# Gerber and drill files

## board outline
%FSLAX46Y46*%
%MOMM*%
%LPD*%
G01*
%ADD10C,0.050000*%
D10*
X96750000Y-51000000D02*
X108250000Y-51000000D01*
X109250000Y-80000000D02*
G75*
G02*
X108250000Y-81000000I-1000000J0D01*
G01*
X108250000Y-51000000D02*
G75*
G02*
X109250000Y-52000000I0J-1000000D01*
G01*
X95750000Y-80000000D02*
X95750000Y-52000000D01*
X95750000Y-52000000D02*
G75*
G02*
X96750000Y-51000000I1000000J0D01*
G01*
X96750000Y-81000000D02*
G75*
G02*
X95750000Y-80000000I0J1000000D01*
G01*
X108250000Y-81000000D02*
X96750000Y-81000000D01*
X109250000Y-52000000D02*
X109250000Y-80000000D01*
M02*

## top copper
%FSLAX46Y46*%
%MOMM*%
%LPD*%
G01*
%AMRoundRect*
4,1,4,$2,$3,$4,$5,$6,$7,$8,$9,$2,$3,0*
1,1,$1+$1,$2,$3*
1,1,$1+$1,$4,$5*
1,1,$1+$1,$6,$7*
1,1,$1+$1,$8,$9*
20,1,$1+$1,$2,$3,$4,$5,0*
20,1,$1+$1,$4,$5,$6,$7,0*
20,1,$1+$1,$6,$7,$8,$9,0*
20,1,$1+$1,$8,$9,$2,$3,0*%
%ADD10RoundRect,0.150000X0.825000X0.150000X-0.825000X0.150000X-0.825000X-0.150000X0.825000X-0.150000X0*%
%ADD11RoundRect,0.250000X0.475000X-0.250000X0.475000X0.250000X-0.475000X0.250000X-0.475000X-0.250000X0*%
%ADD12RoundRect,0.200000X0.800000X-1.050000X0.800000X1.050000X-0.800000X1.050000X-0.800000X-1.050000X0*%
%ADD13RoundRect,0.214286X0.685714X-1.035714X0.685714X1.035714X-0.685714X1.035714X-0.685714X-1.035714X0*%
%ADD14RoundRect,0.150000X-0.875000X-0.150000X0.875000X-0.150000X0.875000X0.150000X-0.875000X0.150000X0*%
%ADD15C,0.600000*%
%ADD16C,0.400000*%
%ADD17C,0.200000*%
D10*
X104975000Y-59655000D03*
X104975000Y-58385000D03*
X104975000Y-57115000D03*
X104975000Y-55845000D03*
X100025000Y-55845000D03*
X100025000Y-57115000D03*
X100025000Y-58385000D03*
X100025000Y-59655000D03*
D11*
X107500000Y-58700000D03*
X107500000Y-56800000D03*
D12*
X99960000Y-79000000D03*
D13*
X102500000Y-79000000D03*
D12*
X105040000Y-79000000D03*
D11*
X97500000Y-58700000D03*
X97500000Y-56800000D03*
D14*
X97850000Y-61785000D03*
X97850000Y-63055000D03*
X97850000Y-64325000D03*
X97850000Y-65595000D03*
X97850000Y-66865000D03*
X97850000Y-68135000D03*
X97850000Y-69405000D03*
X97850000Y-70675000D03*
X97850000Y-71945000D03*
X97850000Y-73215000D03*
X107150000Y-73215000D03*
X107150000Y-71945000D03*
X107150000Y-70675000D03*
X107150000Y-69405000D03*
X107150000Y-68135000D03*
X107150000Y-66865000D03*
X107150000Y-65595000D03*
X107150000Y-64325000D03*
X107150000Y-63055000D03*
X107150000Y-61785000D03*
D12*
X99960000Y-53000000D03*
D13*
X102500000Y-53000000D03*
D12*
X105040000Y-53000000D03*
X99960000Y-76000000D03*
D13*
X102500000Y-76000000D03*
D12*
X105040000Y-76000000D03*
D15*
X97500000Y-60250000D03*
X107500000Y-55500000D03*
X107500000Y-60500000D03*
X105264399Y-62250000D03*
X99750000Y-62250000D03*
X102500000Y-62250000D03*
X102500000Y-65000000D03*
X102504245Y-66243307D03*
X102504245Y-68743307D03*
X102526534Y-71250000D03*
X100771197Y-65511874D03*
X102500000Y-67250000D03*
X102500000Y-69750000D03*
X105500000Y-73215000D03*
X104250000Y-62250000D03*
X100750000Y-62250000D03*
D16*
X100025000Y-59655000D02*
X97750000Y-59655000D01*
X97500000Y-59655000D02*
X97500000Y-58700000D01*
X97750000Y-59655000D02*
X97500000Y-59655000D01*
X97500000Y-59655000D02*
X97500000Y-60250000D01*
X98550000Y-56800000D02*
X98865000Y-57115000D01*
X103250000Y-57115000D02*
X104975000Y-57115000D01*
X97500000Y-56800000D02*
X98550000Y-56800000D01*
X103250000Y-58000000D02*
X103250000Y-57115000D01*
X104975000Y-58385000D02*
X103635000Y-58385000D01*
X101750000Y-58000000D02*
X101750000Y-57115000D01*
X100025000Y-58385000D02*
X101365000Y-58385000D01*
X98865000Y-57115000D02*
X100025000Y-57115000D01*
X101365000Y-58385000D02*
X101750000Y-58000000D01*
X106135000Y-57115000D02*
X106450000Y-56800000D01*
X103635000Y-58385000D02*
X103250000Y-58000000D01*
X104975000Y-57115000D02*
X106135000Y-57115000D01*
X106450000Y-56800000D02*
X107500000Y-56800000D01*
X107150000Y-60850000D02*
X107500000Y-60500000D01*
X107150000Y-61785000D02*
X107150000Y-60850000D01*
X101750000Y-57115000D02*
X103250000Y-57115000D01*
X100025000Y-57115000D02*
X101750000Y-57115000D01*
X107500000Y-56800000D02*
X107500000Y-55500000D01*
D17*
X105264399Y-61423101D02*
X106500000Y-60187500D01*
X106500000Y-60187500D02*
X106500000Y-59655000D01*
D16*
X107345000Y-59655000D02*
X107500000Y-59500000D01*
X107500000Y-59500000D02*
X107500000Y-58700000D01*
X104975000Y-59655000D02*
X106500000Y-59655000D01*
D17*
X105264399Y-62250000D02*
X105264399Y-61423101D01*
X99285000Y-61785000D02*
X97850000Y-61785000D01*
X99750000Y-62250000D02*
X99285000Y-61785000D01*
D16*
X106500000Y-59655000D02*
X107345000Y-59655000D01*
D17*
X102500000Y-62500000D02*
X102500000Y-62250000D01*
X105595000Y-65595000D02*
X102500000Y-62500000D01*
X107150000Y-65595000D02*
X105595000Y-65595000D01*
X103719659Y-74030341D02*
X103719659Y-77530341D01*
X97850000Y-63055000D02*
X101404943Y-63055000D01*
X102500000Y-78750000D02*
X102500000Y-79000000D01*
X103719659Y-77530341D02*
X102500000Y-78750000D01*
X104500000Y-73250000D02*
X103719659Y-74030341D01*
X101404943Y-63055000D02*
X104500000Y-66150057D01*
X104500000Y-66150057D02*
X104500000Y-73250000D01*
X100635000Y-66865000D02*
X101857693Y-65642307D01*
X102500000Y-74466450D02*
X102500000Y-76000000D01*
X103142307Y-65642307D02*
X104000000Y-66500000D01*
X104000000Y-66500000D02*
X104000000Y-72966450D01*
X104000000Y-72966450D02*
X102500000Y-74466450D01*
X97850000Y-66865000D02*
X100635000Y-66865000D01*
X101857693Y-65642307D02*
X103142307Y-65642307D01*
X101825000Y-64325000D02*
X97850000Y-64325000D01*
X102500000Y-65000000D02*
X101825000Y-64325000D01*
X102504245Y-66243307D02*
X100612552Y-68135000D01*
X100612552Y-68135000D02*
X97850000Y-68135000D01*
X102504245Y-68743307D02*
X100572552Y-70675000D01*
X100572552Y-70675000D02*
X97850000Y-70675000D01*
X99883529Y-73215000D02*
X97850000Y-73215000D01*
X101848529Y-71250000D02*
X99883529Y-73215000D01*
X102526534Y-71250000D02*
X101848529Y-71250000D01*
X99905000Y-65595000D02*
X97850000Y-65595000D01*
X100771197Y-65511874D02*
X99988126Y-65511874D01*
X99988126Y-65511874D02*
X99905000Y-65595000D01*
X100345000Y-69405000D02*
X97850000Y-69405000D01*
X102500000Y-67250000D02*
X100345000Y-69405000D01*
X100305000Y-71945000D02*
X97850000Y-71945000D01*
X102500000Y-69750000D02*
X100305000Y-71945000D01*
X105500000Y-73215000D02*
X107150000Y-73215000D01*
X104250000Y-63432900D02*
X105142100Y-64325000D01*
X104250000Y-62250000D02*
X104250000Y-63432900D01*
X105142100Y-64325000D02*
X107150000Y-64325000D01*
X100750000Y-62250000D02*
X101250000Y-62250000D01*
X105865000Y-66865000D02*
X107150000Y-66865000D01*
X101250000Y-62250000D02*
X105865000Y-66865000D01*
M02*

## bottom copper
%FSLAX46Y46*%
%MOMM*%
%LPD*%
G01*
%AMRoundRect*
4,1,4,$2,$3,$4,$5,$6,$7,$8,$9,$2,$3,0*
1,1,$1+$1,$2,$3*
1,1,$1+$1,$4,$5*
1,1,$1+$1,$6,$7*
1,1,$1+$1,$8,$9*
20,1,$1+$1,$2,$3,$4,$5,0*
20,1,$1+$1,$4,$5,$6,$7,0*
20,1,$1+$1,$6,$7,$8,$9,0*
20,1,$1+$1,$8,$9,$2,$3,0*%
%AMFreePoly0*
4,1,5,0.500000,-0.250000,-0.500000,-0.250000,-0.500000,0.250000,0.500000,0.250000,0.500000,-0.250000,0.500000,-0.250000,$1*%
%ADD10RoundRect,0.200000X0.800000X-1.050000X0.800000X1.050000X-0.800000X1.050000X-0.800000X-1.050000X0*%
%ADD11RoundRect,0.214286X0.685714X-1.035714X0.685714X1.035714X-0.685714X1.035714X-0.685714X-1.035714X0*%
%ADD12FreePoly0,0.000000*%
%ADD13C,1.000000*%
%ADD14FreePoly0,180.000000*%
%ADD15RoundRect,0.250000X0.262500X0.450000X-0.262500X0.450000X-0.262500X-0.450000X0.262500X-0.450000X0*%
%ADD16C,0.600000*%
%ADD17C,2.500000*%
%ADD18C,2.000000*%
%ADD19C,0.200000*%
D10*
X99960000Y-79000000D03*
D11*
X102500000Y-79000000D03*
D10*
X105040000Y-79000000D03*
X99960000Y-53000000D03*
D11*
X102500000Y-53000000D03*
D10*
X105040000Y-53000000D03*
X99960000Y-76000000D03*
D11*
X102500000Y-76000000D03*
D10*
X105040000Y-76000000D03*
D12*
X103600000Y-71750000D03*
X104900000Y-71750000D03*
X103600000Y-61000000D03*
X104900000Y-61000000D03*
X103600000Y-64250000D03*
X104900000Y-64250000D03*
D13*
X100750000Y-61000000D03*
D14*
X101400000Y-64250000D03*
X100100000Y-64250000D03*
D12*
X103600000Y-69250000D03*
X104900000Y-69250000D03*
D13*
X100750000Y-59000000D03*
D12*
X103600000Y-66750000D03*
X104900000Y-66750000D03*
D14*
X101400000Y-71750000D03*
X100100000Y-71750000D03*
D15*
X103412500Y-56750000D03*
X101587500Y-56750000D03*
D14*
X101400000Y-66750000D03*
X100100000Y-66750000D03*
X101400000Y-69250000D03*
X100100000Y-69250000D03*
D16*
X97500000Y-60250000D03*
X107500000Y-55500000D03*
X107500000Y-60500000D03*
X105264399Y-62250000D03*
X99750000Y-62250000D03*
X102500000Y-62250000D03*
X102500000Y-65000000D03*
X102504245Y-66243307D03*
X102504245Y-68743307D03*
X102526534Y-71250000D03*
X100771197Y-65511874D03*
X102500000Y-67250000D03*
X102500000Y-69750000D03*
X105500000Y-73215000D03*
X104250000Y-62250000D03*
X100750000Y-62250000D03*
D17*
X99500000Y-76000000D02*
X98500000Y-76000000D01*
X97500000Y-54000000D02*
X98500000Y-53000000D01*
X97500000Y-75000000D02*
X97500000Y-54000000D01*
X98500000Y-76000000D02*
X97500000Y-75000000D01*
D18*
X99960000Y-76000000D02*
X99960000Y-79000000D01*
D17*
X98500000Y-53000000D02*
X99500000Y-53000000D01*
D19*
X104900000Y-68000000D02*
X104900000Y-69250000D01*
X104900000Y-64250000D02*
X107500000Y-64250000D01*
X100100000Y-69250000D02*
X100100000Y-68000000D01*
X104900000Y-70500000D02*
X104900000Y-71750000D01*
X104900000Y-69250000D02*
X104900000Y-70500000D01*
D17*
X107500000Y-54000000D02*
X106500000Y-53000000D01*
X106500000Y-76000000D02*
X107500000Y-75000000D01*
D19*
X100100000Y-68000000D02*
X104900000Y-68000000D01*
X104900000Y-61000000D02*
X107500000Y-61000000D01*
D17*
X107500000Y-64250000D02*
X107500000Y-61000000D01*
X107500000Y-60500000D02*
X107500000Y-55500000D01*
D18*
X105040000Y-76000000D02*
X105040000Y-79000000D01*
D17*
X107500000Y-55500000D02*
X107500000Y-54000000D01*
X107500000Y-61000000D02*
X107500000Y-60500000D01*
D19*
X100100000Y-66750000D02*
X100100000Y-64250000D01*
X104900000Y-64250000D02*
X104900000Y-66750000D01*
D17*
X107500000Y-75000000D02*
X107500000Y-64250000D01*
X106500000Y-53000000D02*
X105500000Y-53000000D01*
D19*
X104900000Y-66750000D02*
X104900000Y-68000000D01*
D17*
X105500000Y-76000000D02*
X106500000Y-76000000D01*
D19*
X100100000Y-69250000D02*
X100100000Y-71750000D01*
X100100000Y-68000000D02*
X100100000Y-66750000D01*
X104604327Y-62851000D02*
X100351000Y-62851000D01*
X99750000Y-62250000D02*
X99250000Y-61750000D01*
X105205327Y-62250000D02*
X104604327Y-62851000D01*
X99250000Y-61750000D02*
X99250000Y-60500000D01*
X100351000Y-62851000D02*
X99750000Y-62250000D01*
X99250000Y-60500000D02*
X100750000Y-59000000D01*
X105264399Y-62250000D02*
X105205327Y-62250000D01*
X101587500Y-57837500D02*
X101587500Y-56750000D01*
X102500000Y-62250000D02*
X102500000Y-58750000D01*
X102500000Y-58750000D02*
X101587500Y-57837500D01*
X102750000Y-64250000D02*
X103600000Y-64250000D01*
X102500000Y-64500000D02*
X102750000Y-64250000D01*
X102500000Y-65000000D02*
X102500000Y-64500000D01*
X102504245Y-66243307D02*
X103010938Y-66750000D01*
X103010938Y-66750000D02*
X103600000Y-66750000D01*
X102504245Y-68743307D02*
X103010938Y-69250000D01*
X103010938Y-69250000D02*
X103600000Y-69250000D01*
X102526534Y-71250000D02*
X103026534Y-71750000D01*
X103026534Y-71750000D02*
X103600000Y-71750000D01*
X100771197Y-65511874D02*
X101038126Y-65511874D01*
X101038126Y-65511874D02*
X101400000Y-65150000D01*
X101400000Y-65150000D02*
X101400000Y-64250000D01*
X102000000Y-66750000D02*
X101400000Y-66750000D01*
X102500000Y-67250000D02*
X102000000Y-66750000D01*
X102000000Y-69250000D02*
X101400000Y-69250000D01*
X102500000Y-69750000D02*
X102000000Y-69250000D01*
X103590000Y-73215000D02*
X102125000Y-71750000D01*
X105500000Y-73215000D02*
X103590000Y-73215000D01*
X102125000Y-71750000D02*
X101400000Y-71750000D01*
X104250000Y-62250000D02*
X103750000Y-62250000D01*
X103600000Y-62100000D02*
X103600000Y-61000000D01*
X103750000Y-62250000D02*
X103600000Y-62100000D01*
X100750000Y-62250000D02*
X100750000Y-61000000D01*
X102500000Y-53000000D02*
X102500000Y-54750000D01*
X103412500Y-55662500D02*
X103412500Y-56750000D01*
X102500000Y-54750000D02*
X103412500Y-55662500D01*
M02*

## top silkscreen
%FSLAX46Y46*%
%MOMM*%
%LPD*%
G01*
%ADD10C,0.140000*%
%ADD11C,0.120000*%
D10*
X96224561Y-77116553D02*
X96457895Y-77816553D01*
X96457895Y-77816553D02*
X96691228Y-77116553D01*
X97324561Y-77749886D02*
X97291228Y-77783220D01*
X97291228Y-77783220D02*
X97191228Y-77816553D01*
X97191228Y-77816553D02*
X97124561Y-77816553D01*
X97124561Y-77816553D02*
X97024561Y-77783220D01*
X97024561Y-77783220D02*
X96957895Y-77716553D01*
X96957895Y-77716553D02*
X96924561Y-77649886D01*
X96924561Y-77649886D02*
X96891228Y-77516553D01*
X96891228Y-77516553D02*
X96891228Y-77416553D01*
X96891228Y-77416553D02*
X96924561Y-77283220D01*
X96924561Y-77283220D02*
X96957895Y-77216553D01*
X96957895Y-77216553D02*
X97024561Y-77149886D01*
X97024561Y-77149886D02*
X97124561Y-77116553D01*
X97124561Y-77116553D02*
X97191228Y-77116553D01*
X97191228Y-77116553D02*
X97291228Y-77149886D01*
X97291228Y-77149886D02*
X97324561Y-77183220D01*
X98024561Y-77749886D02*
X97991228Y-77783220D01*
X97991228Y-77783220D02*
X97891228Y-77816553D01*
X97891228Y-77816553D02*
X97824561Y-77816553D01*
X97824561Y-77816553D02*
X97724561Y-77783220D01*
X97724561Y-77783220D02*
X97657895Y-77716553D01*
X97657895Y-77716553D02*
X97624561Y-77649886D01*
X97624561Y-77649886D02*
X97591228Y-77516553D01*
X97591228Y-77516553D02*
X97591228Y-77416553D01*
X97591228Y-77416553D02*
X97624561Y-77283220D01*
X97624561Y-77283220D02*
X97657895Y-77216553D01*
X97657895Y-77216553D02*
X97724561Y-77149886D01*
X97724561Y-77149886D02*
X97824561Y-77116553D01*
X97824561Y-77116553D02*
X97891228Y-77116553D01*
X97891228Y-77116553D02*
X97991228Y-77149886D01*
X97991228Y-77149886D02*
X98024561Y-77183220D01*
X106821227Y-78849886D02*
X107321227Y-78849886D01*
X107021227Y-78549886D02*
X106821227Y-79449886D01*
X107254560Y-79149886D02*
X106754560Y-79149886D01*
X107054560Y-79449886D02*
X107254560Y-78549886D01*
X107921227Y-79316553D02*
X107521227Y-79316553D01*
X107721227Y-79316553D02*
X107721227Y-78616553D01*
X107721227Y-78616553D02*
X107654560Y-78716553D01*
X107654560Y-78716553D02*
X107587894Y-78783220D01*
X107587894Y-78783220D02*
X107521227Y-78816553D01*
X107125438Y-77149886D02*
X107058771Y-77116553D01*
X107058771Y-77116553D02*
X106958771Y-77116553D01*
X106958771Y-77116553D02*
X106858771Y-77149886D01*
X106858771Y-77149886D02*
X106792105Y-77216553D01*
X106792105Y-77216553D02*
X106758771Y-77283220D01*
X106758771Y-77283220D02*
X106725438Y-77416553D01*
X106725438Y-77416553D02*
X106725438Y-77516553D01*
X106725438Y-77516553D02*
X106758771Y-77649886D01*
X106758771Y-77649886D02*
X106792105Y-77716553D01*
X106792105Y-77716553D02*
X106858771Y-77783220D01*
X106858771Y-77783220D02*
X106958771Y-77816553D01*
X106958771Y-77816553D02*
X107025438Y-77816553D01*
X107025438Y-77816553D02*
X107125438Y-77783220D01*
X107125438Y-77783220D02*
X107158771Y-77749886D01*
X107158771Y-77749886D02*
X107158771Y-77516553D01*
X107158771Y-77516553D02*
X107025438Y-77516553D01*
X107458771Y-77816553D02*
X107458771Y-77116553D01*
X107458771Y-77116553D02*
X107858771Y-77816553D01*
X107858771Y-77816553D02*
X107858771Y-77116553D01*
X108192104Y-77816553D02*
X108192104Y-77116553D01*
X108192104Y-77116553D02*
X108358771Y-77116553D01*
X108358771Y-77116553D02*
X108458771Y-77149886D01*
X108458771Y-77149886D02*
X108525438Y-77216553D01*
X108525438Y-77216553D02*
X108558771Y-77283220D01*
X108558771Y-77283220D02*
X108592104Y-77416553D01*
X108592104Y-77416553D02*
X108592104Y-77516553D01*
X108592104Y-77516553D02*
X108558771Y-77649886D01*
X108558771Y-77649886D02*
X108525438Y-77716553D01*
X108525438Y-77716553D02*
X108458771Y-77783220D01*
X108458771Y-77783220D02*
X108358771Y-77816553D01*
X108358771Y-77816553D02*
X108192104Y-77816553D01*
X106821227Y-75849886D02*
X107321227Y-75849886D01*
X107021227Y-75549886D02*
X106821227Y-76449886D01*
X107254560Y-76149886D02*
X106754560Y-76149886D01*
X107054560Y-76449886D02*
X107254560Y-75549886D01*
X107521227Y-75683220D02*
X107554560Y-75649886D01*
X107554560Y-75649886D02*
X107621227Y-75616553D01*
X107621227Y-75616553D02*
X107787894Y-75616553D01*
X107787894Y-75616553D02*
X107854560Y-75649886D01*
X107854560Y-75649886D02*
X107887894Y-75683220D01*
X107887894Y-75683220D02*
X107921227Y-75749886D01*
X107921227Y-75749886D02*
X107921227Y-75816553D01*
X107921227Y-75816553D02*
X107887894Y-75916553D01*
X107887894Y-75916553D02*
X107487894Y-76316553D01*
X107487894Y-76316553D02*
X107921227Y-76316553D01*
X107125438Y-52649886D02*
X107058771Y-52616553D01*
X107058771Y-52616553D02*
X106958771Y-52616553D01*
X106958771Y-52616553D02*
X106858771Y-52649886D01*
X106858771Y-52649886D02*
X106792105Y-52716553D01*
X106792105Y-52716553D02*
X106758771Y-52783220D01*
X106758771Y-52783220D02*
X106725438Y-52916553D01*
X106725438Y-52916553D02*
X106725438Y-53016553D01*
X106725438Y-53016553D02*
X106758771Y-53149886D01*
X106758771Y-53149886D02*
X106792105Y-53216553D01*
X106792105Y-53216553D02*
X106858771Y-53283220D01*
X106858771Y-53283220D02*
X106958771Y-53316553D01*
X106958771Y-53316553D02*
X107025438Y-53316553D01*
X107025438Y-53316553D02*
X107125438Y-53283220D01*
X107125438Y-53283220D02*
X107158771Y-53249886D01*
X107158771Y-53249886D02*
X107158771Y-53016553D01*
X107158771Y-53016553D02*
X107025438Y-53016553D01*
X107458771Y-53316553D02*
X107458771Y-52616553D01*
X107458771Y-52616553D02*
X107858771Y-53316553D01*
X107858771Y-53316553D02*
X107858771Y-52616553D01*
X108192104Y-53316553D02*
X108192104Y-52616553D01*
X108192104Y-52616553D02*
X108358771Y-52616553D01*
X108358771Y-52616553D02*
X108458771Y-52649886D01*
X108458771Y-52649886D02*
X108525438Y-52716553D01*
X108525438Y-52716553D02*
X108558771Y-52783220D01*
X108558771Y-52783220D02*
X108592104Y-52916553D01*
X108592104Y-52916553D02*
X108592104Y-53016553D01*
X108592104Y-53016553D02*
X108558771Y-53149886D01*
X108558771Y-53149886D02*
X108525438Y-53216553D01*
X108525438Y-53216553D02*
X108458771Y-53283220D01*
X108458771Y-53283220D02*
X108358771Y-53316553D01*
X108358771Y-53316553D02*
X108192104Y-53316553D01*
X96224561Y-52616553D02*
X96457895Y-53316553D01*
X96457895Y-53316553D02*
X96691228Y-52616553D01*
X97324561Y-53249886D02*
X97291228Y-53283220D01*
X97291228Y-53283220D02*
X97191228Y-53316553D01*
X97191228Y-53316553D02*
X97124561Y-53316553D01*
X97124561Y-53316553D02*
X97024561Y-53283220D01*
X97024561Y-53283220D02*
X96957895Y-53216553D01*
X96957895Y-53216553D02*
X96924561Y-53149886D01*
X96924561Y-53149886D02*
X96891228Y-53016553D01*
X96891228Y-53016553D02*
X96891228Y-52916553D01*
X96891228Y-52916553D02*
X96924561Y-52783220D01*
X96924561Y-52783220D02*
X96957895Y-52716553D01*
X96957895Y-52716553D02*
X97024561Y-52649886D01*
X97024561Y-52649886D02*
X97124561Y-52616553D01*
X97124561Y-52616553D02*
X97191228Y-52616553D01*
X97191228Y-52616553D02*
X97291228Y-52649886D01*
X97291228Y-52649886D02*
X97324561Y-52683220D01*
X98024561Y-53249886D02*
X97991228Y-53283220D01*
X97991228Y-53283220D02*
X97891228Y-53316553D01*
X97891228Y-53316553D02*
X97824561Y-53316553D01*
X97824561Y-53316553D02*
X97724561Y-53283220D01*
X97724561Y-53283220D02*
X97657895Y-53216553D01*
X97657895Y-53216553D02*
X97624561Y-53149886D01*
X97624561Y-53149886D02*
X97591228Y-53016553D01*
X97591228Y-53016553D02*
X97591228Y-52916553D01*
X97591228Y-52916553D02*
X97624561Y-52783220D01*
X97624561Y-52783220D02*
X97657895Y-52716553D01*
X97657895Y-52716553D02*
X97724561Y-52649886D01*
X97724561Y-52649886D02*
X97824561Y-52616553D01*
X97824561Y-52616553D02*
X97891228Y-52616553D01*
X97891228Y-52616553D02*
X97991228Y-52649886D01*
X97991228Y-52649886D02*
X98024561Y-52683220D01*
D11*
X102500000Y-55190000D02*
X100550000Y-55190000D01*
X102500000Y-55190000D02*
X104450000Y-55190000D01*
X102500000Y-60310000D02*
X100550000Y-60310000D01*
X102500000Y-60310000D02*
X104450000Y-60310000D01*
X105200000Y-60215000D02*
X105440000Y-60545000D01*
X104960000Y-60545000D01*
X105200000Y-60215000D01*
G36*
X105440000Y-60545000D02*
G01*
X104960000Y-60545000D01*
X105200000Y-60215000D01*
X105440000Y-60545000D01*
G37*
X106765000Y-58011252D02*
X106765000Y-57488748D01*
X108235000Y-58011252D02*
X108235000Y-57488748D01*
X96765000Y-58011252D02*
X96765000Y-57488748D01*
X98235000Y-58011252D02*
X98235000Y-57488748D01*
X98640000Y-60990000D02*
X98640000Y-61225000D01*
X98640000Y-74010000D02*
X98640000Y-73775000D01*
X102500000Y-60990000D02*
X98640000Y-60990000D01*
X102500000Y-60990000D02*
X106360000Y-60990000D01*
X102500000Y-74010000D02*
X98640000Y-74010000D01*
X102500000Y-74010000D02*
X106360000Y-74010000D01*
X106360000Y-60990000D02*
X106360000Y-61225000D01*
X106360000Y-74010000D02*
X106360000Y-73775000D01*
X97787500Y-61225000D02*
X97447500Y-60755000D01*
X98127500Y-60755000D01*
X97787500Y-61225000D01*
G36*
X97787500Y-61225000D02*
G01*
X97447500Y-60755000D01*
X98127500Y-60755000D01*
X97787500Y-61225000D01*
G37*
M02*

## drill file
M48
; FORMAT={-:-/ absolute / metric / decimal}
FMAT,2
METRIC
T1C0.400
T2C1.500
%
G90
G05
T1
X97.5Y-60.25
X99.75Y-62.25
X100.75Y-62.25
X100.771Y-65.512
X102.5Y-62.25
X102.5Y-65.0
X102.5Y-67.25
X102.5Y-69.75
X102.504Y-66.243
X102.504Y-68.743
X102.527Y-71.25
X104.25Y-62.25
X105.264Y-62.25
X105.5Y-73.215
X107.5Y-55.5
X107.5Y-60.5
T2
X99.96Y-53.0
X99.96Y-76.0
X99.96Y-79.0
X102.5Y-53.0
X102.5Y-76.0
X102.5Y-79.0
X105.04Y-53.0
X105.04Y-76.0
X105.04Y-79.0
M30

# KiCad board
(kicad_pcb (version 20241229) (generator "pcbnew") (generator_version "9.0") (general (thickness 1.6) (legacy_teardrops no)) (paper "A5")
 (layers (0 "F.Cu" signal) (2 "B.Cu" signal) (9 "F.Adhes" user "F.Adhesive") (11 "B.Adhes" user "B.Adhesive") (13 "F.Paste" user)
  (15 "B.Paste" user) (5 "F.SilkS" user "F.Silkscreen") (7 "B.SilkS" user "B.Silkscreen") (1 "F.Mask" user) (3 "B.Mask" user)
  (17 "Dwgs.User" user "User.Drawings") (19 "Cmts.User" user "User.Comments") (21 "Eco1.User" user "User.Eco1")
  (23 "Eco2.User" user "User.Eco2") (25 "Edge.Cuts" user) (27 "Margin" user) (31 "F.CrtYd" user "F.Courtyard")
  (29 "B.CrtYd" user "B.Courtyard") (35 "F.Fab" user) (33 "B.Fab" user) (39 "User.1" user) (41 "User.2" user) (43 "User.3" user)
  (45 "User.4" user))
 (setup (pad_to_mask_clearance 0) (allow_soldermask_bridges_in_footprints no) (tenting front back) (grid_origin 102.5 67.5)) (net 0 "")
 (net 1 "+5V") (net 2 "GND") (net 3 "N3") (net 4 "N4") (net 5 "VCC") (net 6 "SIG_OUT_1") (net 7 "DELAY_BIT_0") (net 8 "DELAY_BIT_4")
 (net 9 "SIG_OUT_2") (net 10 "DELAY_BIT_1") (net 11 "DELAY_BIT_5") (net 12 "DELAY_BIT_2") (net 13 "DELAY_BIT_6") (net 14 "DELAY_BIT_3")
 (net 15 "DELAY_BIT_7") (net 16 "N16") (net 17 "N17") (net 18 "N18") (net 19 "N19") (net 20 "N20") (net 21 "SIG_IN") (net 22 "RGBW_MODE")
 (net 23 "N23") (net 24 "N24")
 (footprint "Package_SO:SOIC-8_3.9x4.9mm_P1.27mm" (layer "F.Cu") (at 102.5 57.75 180)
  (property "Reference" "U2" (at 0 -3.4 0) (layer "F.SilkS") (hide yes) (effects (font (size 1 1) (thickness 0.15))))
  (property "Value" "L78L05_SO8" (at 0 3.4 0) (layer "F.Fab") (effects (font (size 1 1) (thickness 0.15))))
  (fp_line (start 0 2.56) (end 1.95 2.56) (stroke (width 0.12) (type solid)) (layer "F.SilkS"))
  (fp_line (start 0 2.56) (end -1.95 2.56) (stroke (width 0.12) (type solid)) (layer "F.SilkS"))
  (fp_line (start 0 -2.56) (end 1.95 -2.56) (stroke (width 0.12) (type solid)) (layer "F.SilkS"))
  (fp_line (start 0 -2.56) (end -1.95 -2.56) (stroke (width 0.12) (type solid)) (layer "F.SilkS"))
  (fp_poly (pts (xy -2.7 -2.465) (xy -2.94 -2.795) (xy -2.46 -2.795)) (stroke (width 0.12) (type solid)) (fill yes) (layer "F.SilkS"))
  (pad "1" smd roundrect (at -2.475 -1.905 180) (size 1.95 0.6) (layers "F.Cu" "F.Mask" "F.Paste") (roundrect_rratio 0.25) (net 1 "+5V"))
  (pad "2" smd roundrect (at -2.475 -0.635 180) (size 1.95 0.6) (layers "F.Cu" "F.Mask" "F.Paste") (roundrect_rratio 0.25) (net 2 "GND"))
  (pad "3" smd roundrect (at -2.475 0.635 180) (size 1.95 0.6) (layers "F.Cu" "F.Mask" "F.Paste") (roundrect_rratio 0.25) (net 2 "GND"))
  (pad "4" smd roundrect (at -2.475 1.905 180) (size 1.95 0.6) (layers "F.Cu" "F.Mask" "F.Paste") (roundrect_rratio 0.25) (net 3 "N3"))
  (pad "5" smd roundrect (at 2.475 1.905 180) (size 1.95 0.6) (layers "F.Cu" "F.Mask" "F.Paste") (roundrect_rratio 0.25) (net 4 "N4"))
  (pad "6" smd roundrect (at 2.475 0.635 180) (size 1.95 0.6) (layers "F.Cu" "F.Mask" "F.Paste") (roundrect_rratio 0.25) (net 2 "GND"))
  (pad "7" smd roundrect (at 2.475 -0.635 180) (size 1.95 0.6) (layers "F.Cu" "F.Mask" "F.Paste") (roundrect_rratio 0.25) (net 2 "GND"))
  (pad "8" smd roundrect (at 2.475 -1.905 180) (size 1.95 0.6) (layers "F.Cu" "F.Mask" "F.Paste") (roundrect_rratio 0.25) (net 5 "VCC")))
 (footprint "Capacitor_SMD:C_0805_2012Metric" (layer "F.Cu") (at 107.5 57.75 90)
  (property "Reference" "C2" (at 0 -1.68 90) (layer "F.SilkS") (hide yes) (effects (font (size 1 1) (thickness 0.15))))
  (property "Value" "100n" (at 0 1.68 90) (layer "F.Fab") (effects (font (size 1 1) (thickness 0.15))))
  (fp_line (start -0.261252 -0.735) (end 0.261252 -0.735) (stroke (width 0.12) (type solid)) (layer "F.SilkS"))
  (fp_line (start -0.261252 0.735) (end 0.261252 0.735) (stroke (width 0.12) (type solid)) (layer "F.SilkS"))
  (pad "1" smd roundrect (at -0.95 0 90) (size 1 1.45) (layers "F.Cu" "F.Mask" "F.Paste") (roundrect_rratio 0.25) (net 1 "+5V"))
  (pad "2" smd roundrect (at 0.95 0 90) (size 1 1.45) (layers "F.Cu" "F.Mask" "F.Paste") (roundrect_rratio 0.25) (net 2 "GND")))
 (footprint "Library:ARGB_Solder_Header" (layer "F.Cu") (at 99.96 79 90)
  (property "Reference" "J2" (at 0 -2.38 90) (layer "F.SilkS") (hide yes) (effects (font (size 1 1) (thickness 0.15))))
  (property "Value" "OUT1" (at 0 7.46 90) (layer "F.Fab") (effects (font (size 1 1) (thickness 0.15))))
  (pad "1" thru_hole roundrect (at 0 0 90) (size 2.5 2) (drill 1.5) (layers "*.Cu" "*.Mask") (remove_unused_layers no)
   (roundrect_rratio 0.1) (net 5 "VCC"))
  (pad "2" thru_hole roundrect (at 0 2.54 90) (size 2.5 1.8) (drill 1.5) (layers "*.Cu" "*.Mask") (remove_unused_layers no)
   (roundrect_rratio 0.119047619) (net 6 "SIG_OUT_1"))
  (pad "3" thru_hole roundrect (at 0 5.08 90) (size 2.5 2) (drill 1.5) (layers "*.Cu" "*.Mask") (remove_unused_layers no)
   (roundrect_rratio 0.1) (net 2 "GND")))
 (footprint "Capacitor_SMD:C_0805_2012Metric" (layer "F.Cu") (at 97.5 57.75 90)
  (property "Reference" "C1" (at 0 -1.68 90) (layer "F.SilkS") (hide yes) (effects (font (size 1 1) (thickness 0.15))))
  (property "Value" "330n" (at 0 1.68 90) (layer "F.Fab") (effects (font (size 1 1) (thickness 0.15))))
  (fp_line (start -0.261252 -0.735) (end 0.261252 -0.735) (stroke (width 0.12) (type solid)) (layer "F.SilkS"))
  (fp_line (start -0.261252 0.735) (end 0.261252 0.735) (stroke (width 0.12) (type solid)) (layer "F.SilkS"))
  (pad "1" smd roundrect (at -0.95 0 90) (size 1 1.45) (layers "F.Cu" "F.Mask" "F.Paste") (roundrect_rratio 0.25) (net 5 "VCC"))
  (pad "2" smd roundrect (at 0.95 0 90) (size 1 1.45) (layers "F.Cu" "F.Mask" "F.Paste") (roundrect_rratio 0.25) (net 2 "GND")))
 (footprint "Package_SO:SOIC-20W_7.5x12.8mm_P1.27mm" (layer "F.Cu") (at 102.5 67.5)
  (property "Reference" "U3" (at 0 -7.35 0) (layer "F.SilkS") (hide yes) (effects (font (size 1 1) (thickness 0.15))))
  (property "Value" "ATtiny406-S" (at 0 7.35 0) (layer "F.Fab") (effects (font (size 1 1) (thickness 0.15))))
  (fp_line (start -3.86 -6.51) (end -3.86 -6.275) (stroke (width 0.12) (type solid)) (layer "F.SilkS"))
  (fp_line (start -3.86 6.51) (end -3.86 6.275) (stroke (width 0.12) (type solid)) (layer "F.SilkS"))
  (fp_line (start 0 -6.51) (end -3.86 -6.51) (stroke (width 0.12) (type solid)) (layer "F.SilkS"))
  (fp_line (start 0 -6.51) (end 3.86 -6.51) (stroke (width 0.12) (type solid)) (layer "F.SilkS"))
  (fp_line (start 0 6.51) (end -3.86 6.51) (stroke (width 0.12) (type solid)) (layer "F.SilkS"))
  (fp_line (start 0 6.51) (end 3.86 6.51) (stroke (width 0.12) (type solid)) (layer "F.SilkS"))
  (fp_line (start 3.86 -6.51) (end 3.86 -6.275) (stroke (width 0.12) (type solid)) (layer "F.SilkS"))
  (fp_line (start 3.86 6.51) (end 3.86 6.275) (stroke (width 0.12) (type solid)) (layer "F.SilkS"))
  (fp_poly
   (pts (xy -4.7125 -6.275) (xy -5.0525 -6.745) (xy -4.3725 -6.745)) (stroke (width 0.12) (type solid)) (fill yes) (layer "F.SilkS"))
  (pad "1" smd roundrect (at -4.65 -5.715) (size 2.05 0.6) (layers "F.Cu" "F.Mask" "F.Paste") (roundrect_rratio 0.25) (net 1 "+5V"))
  (pad "2" smd roundrect (at -4.65 -4.445) (size 2.05 0.6) (layers "F.Cu" "F.Mask" "F.Paste") (roundrect_rratio 0.25) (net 6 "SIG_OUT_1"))
  (pad "3" smd roundrect (at -4.65 -3.175) (size 2.05 0.6) (layers "F.Cu" "F.Mask" "F.Paste") (roundrect_rratio 0.25) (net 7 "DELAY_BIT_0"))
  (pad "4" smd roundrect (at -4.65 -1.905) (size 2.05 0.6) (layers "F.Cu" "F.Mask" "F.Paste") (roundrect_rratio 0.25) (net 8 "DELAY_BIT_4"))
  (pad "5" smd roundrect (at -4.65 -0.635) (size 2.05 0.6) (layers "F.Cu" "F.Mask" "F.Paste") (roundrect_rratio 0.25) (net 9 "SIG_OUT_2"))
  (pad "6" smd roundrect (at -4.65 0.635) (size 2.05 0.6) (layers "F.Cu" "F.Mask" "F.Paste") (roundrect_rratio 0.25) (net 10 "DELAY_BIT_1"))
  (pad "7" smd roundrect (at -4.65 1.905) (size 2.05 0.6) (layers "F.Cu" "F.Mask" "F.Paste") (roundrect_rratio 0.25) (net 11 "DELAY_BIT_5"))
  (pad "8" smd roundrect (at -4.65 3.175) (size 2.05 0.6) (layers "F.Cu" "F.Mask" "F.Paste") (roundrect_rratio 0.25) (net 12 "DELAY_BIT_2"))
  (pad "9" smd roundrect (at -4.65 4.445) (size 2.05 0.6) (layers "F.Cu" "F.Mask" "F.Paste") (roundrect_rratio 0.25) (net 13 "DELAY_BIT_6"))
  (pad "10" smd roundrect (at -4.65 5.715) (size 2.05 0.6) (layers "F.Cu" "F.Mask" "F.Paste") (roundrect_rratio 0.25) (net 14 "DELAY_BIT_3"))
  (pad "11" smd roundrect (at 4.65 5.715) (size 2.05 0.6) (layers "F.Cu" "F.Mask" "F.Paste") (roundrect_rratio 0.25) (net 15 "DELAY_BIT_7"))
  (pad "12" smd roundrect (at 4.65 4.445) (size 2.05 0.6) (layers "F.Cu" "F.Mask" "F.Paste") (roundrect_rratio 0.25) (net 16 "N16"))
  (pad "13" smd roundrect (at 4.65 3.175) (size 2.05 0.6) (layers "F.Cu" "F.Mask" "F.Paste") (roundrect_rratio 0.25) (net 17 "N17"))
  (pad "14" smd roundrect (at 4.65 1.905) (size 2.05 0.6) (layers "F.Cu" "F.Mask" "F.Paste") (roundrect_rratio 0.25) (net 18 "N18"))
  (pad "15" smd roundrect (at 4.65 0.635) (size 2.05 0.6) (layers "F.Cu" "F.Mask" "F.Paste") (roundrect_rratio 0.25) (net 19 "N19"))
  (pad "16" smd roundrect (at 4.65 -0.635) (size 2.05 0.6) (layers "F.Cu" "F.Mask" "F.Paste") (roundrect_rratio 0.25) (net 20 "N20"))
  (pad "17" smd roundrect (at 4.65 -1.905) (size 2.05 0.6) (layers "F.Cu" "F.Mask" "F.Paste") (roundrect_rratio 0.25) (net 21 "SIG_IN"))
  (pad "18" smd roundrect (at 4.65 -3.175) (size 2.05 0.6) (layers "F.Cu" "F.Mask" "F.Paste") (roundrect_rratio 0.25) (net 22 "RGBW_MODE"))
  (pad "19" smd roundrect (at 4.65 -4.445) (size 2.05 0.6) (layers "F.Cu" "F.Mask" "F.Paste") (roundrect_rratio 0.25) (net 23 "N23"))
  (pad "20" smd roundrect (at 4.65 -5.715) (size 2.05 0.6) (layers "F.Cu" "F.Mask" "F.Paste") (roundrect_rratio 0.25) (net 2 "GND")))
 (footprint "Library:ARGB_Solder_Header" (layer "F.Cu") (at 99.96 53 90)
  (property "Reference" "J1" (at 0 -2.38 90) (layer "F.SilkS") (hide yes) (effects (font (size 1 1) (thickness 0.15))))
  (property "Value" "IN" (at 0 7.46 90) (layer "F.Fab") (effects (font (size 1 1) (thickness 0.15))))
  (pad "1" thru_hole roundrect (at 0 0 90) (size 2.5 2) (drill 1.5) (layers "*.Cu" "*.Mask") (remove_unused_layers no)
   (roundrect_rratio 0.1) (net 5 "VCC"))
  (pad "2" thru_hole roundrect (at 0 2.54 90) (size 2.5 1.8) (drill 1.5) (layers "*.Cu" "*.Mask") (remove_unused_layers no)
   (roundrect_rratio 0.119047619) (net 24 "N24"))
  (pad "3" thru_hole roundrect (at 0 5.08 90) (size 2.5 2) (drill 1.5) (layers "*.Cu" "*.Mask") (remove_unused_layers no)
   (roundrect_rratio 0.1) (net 2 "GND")))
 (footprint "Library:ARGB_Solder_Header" (layer "F.Cu") (at 99.96 76 90)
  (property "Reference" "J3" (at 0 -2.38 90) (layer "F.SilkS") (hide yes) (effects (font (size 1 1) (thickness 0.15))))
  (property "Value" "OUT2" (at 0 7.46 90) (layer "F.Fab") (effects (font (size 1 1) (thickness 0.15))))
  (pad "1" thru_hole roundrect (at 0 0 90) (size 2.5 2) (drill 1.5) (layers "*.Cu" "*.Mask") (remove_unused_layers no)
   (roundrect_rratio 0.1) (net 5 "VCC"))
  (pad "2" thru_hole roundrect (at 0 2.54 90) (size 2.5 1.8) (drill 1.5) (layers "*.Cu" "*.Mask") (remove_unused_layers no)
   (roundrect_rratio 0.119047619) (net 9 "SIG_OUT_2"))
  (pad "3" thru_hole roundrect (at 0 5.08 90) (size 2.5 2) (drill 1.5) (layers "*.Cu" "*.Mask") (remove_unused_layers no)
   (roundrect_rratio 0.1) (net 2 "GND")))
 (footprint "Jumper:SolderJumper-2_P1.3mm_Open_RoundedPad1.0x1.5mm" (layer "B.Cu") (at 104.25 71.75)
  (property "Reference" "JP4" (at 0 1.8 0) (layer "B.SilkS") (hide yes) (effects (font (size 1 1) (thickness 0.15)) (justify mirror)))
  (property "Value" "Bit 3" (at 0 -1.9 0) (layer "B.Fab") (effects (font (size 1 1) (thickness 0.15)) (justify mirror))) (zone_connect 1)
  (pad "1" smd custom (at -0.65 0) (size 1 0.5) (layers "B.Cu" "B.Mask") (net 14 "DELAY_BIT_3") (zone_connect 2) (thermal_bridge_angle 45)
   (options (clearance outline) (anchor rect)) (primitives))
  (pad "2" smd custom (at 0.65 0) (size 1 0.5) (layers "B.Cu" "B.Mask") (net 2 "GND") (zone_connect 2) (thermal_bridge_angle 45)
   (options (clearance outline) (anchor rect)) (primitives)))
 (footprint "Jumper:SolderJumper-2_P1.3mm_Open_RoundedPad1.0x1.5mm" (layer "B.Cu") (at 104.25 61)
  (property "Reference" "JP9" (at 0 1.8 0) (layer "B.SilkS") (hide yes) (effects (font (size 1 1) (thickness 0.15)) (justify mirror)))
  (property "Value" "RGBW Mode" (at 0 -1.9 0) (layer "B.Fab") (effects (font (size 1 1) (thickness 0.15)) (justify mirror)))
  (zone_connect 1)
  (pad "1" smd custom (at -0.65 0) (size 1 0.5) (layers "B.Cu" "B.Mask") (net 22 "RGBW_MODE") (zone_connect 2) (thermal_bridge_angle 45)
   (options (clearance outline) (anchor rect)) (primitives))
  (pad "2" smd custom (at 0.65 0) (size 1 0.5) (layers "B.Cu" "B.Mask") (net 2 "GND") (zone_connect 2) (thermal_bridge_angle 45)
   (options (clearance outline) (anchor rect)) (primitives)))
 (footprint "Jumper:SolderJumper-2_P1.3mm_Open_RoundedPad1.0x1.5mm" (layer "B.Cu") (at 104.25 64.25)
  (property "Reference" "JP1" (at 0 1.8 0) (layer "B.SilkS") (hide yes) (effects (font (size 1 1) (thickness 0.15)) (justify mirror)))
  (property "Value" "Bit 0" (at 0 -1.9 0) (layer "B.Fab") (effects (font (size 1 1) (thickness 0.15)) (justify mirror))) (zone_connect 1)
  (pad "1" smd custom (at -0.65 0) (size 1 0.5) (layers "B.Cu" "B.Mask") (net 7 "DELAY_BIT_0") (zone_connect 2) (thermal_bridge_angle 45)
   (options (clearance outline) (anchor rect)) (primitives))
  (pad "2" smd custom (at 0.65 0) (size 1 0.5) (layers "B.Cu" "B.Mask") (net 2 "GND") (zone_connect 2) (thermal_bridge_angle 45)
   (options (clearance outline) (anchor rect)) (primitives)))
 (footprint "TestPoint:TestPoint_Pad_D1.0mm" (layer "B.Cu") (at 100.75 61 90)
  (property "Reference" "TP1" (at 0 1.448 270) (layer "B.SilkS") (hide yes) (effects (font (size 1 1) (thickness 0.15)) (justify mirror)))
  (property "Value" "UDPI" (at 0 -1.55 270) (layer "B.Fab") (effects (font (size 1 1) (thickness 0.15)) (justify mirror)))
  (pad "1" smd circle (at 0 0 90) (size 1 1) (layers "B.Cu" "B.Mask") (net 20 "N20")))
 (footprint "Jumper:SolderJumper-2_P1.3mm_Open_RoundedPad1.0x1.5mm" (layer "B.Cu") (at 100.75 64.25 180)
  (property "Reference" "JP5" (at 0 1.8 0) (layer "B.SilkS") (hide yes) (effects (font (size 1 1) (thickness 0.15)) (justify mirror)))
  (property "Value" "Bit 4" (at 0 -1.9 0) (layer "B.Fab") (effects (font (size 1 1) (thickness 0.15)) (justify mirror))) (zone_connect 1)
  (pad "1" smd custom (at -0.65 0 180) (size 1 0.5) (layers "B.Cu" "B.Mask") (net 8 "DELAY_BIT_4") (zone_connect 2)
   (thermal_bridge_angle 45) (options (clearance outline) (anchor rect)) (primitives))
  (pad "2" smd custom (at 0.65 0 180) (size 1 0.5) (layers "B.Cu" "B.Mask") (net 2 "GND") (zone_connect 2) (thermal_bridge_angle 45)
   (options (clearance outline) (anchor rect)) (primitives)))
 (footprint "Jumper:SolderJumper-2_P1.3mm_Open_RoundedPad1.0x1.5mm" (layer "B.Cu") (at 104.25 69.25)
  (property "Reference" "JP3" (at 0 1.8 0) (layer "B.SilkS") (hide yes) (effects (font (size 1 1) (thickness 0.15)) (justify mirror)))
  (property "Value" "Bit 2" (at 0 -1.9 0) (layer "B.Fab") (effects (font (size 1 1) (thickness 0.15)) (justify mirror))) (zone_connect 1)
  (pad "1" smd custom (at -0.65 0) (size 1 0.5) (layers "B.Cu" "B.Mask") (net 12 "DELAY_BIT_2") (zone_connect 2) (thermal_bridge_angle 45)
   (options (clearance outline) (anchor rect)) (primitives))
  (pad "2" smd custom (at 0.65 0) (size 1 0.5) (layers "B.Cu" "B.Mask") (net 2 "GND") (zone_connect 2) (thermal_bridge_angle 45)
   (options (clearance outline) (anchor rect)) (primitives)))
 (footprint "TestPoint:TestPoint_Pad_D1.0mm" (layer "B.Cu") (at 100.75 59 180)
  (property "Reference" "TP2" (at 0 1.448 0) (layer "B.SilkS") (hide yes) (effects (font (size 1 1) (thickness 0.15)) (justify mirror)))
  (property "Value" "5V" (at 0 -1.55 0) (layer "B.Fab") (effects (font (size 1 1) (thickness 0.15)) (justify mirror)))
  (pad "1" smd circle (at 0 0 180) (size 1 1) (layers "B.Cu" "B.Mask") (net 1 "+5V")))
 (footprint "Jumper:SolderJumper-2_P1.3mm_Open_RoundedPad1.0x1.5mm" (layer "B.Cu") (at 104.25 66.75)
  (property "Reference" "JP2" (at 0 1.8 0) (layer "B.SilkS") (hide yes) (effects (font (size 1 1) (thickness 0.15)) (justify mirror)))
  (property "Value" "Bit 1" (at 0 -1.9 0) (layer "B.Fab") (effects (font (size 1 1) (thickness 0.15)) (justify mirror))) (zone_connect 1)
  (pad "1" smd custom (at -0.65 0) (size 1 0.5) (layers "B.Cu" "B.Mask") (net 10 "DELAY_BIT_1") (zone_connect 2) (thermal_bridge_angle 45)
   (options (clearance outline) (anchor rect)) (primitives))
  (pad "2" smd custom (at 0.65 0) (size 1 0.5) (layers "B.Cu" "B.Mask") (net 2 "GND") (zone_connect 2) (thermal_bridge_angle 45)
   (options (clearance outline) (anchor rect)) (primitives)))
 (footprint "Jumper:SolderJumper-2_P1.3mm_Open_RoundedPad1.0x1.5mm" (layer "B.Cu") (at 100.75 71.75 180)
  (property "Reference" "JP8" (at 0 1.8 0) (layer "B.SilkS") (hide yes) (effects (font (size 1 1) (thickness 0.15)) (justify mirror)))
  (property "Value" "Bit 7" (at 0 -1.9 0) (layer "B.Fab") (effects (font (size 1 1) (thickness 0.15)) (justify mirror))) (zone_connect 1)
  (pad "1" smd custom (at -0.65 0 180) (size 1 0.5) (layers "B.Cu" "B.Mask") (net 15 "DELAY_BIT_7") (zone_connect 2)
   (thermal_bridge_angle 45) (options (clearance outline) (anchor rect)) (primitives))
  (pad "2" smd custom (at 0.65 0 180) (size 1 0.5) (layers "B.Cu" "B.Mask") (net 2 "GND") (zone_connect 2) (thermal_bridge_angle 45)
   (options (clearance outline) (anchor rect)) (primitives)))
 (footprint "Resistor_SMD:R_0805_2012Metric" (layer "B.Cu") (at 102.5 56.75 180)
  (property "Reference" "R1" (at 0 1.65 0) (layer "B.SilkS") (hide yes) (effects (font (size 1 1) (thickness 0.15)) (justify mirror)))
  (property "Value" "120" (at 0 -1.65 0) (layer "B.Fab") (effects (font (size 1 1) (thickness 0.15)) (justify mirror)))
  (pad "1" smd roundrect (at -0.9125 0 180) (size 1.025 1.4) (layers "B.Cu" "B.Mask" "B.Paste") (roundrect_rratio 0.243902) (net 24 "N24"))
  (pad "2" smd roundrect (at 0.9125 0 180) (size 1.025 1.4) (layers "B.Cu" "B.Mask" "B.Paste") (roundrect_rratio 0.243902) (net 21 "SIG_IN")))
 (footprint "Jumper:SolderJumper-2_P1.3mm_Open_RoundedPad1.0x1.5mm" (layer "B.Cu") (at 100.75 66.75 180)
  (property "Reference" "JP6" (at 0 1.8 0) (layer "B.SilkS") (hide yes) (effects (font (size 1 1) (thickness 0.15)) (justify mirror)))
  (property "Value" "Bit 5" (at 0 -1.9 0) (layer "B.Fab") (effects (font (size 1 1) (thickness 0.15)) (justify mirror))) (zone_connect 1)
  (pad "1" smd custom (at -0.65 0 180) (size 1 0.5) (layers "B.Cu" "B.Mask") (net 11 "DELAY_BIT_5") (zone_connect 2)
   (thermal_bridge_angle 45) (options (clearance outline) (anchor rect)) (primitives))
  (pad "2" smd custom (at 0.65 0 180) (size 1 0.5) (layers "B.Cu" "B.Mask") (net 2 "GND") (zone_connect 2) (thermal_bridge_angle 45)
   (options (clearance outline) (anchor rect)) (primitives)))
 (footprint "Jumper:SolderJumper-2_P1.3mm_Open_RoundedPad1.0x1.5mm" (layer "B.Cu") (at 100.75 69.25 180)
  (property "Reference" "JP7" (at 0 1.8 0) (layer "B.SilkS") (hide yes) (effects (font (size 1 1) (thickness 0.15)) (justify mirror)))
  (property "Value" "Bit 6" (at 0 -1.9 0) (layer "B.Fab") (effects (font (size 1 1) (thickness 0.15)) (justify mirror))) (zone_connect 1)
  (pad "1" smd custom (at -0.65 0 180) (size 1 0.5) (layers "B.Cu" "B.Mask") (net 13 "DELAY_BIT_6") (zone_connect 2)
   (thermal_bridge_angle 45) (options (clearance outline) (anchor rect)) (primitives))
  (pad "2" smd custom (at 0.65 0 180) (size 1 0.5) (layers "B.Cu" "B.Mask") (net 2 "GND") (zone_connect 2) (thermal_bridge_angle 45)
   (options (clearance outline) (anchor rect)) (primitives)))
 (gr_line (start 96.75 51) (end 108.25 51) (stroke (width 0.05) (type default)) (layer "Edge.Cuts"))
 (gr_arc (start 109.25 80) (mid 108.957107 80.707107) (end 108.25 81) (stroke (width 0.05) (type default)) (layer "Edge.Cuts"))
 (gr_arc (start 108.25 51) (mid 108.957107 51.292893) (end 109.25 52) (stroke (width 0.05) (type default)) (layer "Edge.Cuts"))
 (gr_line (start 95.75 80) (end 95.75 52) (stroke (width 0.05) (type default)) (layer "Edge.Cuts"))
 (gr_arc (start 95.75 52) (mid 96.042893 51.292893) (end 96.75 51) (stroke (width 0.05) (type default)) (layer "Edge.Cuts"))
 (gr_arc (start 96.75 81) (mid 96.042893 80.707107) (end 95.75 80) (stroke (width 0.05) (type default)) (layer "Edge.Cuts"))
 (gr_line (start 108.25 81) (end 96.75 81) (stroke (width 0.05) (type default)) (layer "Edge.Cuts"))
 (gr_line (start 109.25 52) (end 109.25 80) (stroke (width 0.05) (type default)) (layer "Edge.Cuts"))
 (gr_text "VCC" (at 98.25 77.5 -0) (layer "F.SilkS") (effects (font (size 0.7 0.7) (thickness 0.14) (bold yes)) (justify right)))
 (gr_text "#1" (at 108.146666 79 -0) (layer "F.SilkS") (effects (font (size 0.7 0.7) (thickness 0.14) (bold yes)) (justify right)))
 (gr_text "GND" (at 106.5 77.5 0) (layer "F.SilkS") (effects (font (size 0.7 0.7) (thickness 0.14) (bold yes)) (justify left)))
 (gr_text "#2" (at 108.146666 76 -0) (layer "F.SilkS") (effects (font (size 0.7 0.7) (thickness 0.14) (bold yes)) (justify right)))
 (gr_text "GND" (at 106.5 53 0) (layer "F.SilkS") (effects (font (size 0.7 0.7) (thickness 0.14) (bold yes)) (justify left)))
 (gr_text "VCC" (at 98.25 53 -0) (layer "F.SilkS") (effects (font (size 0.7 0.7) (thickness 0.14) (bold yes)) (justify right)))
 (segment (start 100.025 59.655) (end 97.75 59.655) (width 0.4) (layer "F.Cu") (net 5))
 (segment (start 97.5 59.655) (end 97.5 58.7) (width 0.4) (layer "F.Cu") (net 5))
 (segment (start 97.75 59.655) (end 97.5 59.655) (width 0.4) (layer "F.Cu") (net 5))
 (segment (start 97.5 59.655) (end 97.5 60.25) (width 0.4) (layer "F.Cu") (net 5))
 (via (at 97.5 60.25) (size 0.6) (drill 0.4) (layers "F.Cu" "B.Cu") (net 5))
 (segment (start 99.5 76) (end 98.5 76) (width 2.5) (layer "B.Cu") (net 5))
 (segment (start 97.5 54) (end 98.5 53) (width 2.5) (layer "B.Cu") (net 5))
 (segment (start 97.5 75) (end 97.5 54) (width 2.5) (layer "B.Cu") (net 5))
 (segment (start 98.5 76) (end 97.5 75) (width 2.5) (layer "B.Cu") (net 5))
 (segment (start 99.96 76) (end 99.96 79) (width 2) (layer "B.Cu") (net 5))
 (segment (start 98.5 53) (end 99.5 53) (width 2.5) (layer "B.Cu") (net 5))
 (segment (start 98.55 56.8) (end 98.865 57.115) (width 0.4) (layer "F.Cu") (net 2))
 (segment (start 103.25 57.115) (end 104.975 57.115) (width 0.4) (layer "F.Cu") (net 2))
 (segment (start 97.5 56.8) (end 98.55 56.8) (width 0.4) (layer "F.Cu") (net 2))
 (segment (start 103.25 58) (end 103.25 57.115) (width 0.4) (layer "F.Cu") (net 2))
 (segment (start 104.975 58.385) (end 103.635 58.385) (width 0.4) (layer "F.Cu") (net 2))
 (segment (start 101.75 58) (end 101.75 57.115) (width 0.4) (layer "F.Cu") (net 2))
 (segment (start 100.025 58.385) (end 101.365 58.385) (width 0.4) (layer "F.Cu") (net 2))
 (segment (start 98.865 57.115) (end 100.025 57.115) (width 0.4) (layer "F.Cu") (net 2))
 (segment (start 101.365 58.385) (end 101.75 58) (width 0.4) (layer "F.Cu") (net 2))
 (segment (start 106.135 57.115) (end 106.45 56.8) (width 0.4) (layer "F.Cu") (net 2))
 (segment (start 103.635 58.385) (end 103.25 58) (width 0.4) (layer "F.Cu") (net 2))
 (segment (start 104.975 57.115) (end 106.135 57.115) (width 0.4) (layer "F.Cu") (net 2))
 (segment (start 106.45 56.8) (end 107.5 56.8) (width 0.4) (layer "F.Cu") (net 2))
 (segment (start 107.15 60.85) (end 107.5 60.5) (width 0.4) (layer "F.Cu") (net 2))
 (segment (start 107.15 61.785) (end 107.15 60.85) (width 0.4) (layer "F.Cu") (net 2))
 (segment (start 101.75 57.115) (end 103.25 57.115) (width 0.4) (layer "F.Cu") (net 2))
 (segment (start 100.025 57.115) (end 101.75 57.115) (width 0.4) (layer "F.Cu") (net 2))
 (segment (start 107.5 56.8) (end 107.5 55.5) (width 0.4) (layer "F.Cu") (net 2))
 (via (at 107.5 55.5) (size 0.6) (drill 0.4) (layers "F.Cu" "B.Cu") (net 2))
 (via (at 107.5 60.5) (size 0.6) (drill 0.4) (layers "F.Cu" "B.Cu") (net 2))
 (segment (start 104.9 68) (end 104.9 69.25) (width 0.2) (layer "B.Cu") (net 2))
 (segment (start 104.9 64.25) (end 107.5 64.25) (width 0.2) (layer "B.Cu") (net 2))
 (segment (start 100.1 69.25) (end 100.1 68) (width 0.2) (layer "B.Cu") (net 2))
 (segment (start 104.9 70.5) (end 104.9 71.75) (width 0.2) (layer "B.Cu") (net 2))
 (segment (start 104.9 69.25) (end 104.9 70.5) (width 0.2) (layer "B.Cu") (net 2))
 (segment (start 107.5 54) (end 106.5 53) (width 2.5) (layer "B.Cu") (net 2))
 (segment (start 106.5 76) (end 107.5 75) (width 2.5) (layer "B.Cu") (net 2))
 (segment (start 100.1 68) (end 104.9 68) (width 0.2) (layer "B.Cu") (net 2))
 (segment (start 104.9 61) (end 107.5 61) (width 0.2) (layer "B.Cu") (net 2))
 (segment (start 107.5 64.25) (end 107.5 61) (width 2.5) (layer "B.Cu") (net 2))
 (segment (start 107.5 60.5) (end 107.5 55.5) (width 2.5) (layer "B.Cu") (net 2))
 (segment (start 105.04 76) (end 105.04 79) (width 2) (layer "B.Cu") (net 2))
 (segment (start 107.5 55.5) (end 107.5 54) (width 2.5) (layer "B.Cu") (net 2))
 (segment (start 107.5 61) (end 107.5 60.5) (width 2.5) (layer "B.Cu") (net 2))
 (segment (start 100.1 66.75) (end 100.1 64.25) (width 0.2) (layer "B.Cu") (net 2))
 (segment (start 104.9 64.25) (end 104.9 66.75) (width 0.2) (layer "B.Cu") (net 2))
 (segment (start 107.5 75) (end 107.5 64.25) (width 2.5) (layer "B.Cu") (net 2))
 (segment (start 106.5 53) (end 105.5 53) (width 2.5) (layer "B.Cu") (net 2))
 (segment (start 104.9 66.75) (end 104.9 68) (width 0.2) (layer "B.Cu") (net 2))
 (segment (start 105.5 76) (end 106.5 76) (width 2.5) (layer "B.Cu") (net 2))
 (segment (start 100.1 69.25) (end 100.1 71.75) (width 0.2) (layer "B.Cu") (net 2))
 (segment (start 100.1 68) (end 100.1 66.75) (width 0.2) (layer "B.Cu") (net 2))
 (segment (start 105.264399 61.423101) (end 106.5 60.1875) (width 0.2) (layer "F.Cu") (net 1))
 (segment (start 106.5 60.1875) (end 106.5 59.655) (width 0.2) (layer "F.Cu") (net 1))
 (segment (start 107.345 59.655) (end 107.5 59.5) (width 0.4) (layer "F.Cu") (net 1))
 (segment (start 107.5 59.5) (end 107.5 58.7) (width 0.4) (layer "F.Cu") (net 1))
 (segment (start 104.975 59.655) (end 106.5 59.655) (width 0.4) (layer "F.Cu") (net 1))
 (segment (start 105.264399 62.25) (end 105.264399 61.423101) (width 0.2) (layer "F.Cu") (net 1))
 (segment (start 99.285 61.785) (end 97.85 61.785) (width 0.2) (layer "F.Cu") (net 1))
 (segment (start 99.75 62.25) (end 99.285 61.785) (width 0.2) (layer "F.Cu") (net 1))
 (segment (start 106.5 59.655) (end 107.345 59.655) (width 0.4) (layer "F.Cu") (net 1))
 (via (at 105.264399 62.25) (size 0.6) (drill 0.4) (layers "F.Cu" "B.Cu") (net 1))
 (via (at 99.75 62.25) (size 0.6) (drill 0.4) (layers "F.Cu" "B.Cu") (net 1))
 (segment (start 104.604327 62.851) (end 100.351 62.851) (width 0.2) (layer "B.Cu") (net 1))
 (segment (start 99.75 62.25) (end 99.25 61.75) (width 0.2) (layer "B.Cu") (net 1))
 (segment (start 105.205327 62.25) (end 104.604327 62.851) (width 0.2) (layer "B.Cu") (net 1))
 (segment (start 99.25 61.75) (end 99.25 60.5) (width 0.2) (layer "B.Cu") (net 1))
 (segment (start 100.351 62.851) (end 99.75 62.25) (width 0.2) (layer "B.Cu") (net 1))
 (segment (start 99.25 60.5) (end 100.75 59) (width 0.2) (layer "B.Cu") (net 1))
 (segment (start 105.264399 62.25) (end 105.205327 62.25) (width 0.2) (layer "B.Cu") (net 1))
 (segment (start 102.5 62.5) (end 102.5 62.25) (width 0.2) (layer "F.Cu") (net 21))
 (segment (start 105.595 65.595) (end 102.5 62.5) (width 0.2) (layer "F.Cu") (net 21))
 (segment (start 107.15 65.595) (end 105.595 65.595) (width 0.2) (layer "F.Cu") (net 21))
 (via (at 102.5 62.25) (size 0.6) (drill 0.4) (layers "F.Cu" "B.Cu") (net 21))
 (segment (start 101.5875 57.8375) (end 101.5875 56.75) (width 0.2) (layer "B.Cu") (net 21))
 (segment (start 102.5 62.25) (end 102.5 58.75) (width 0.2) (layer "B.Cu") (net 21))
 (segment (start 102.5 58.75) (end 101.5875 57.8375) (width 0.2) (layer "B.Cu") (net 21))
 (segment (start 103.719659 74.030341) (end 103.719659 77.530341) (width 0.2) (layer "F.Cu") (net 6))
 (segment (start 97.85 63.055) (end 101.404943 63.055) (width 0.2) (layer "F.Cu") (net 6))
 (segment (start 102.5 78.75) (end 102.5 79) (width 0.2) (layer "F.Cu") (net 6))
 (segment (start 103.719659 77.530341) (end 102.5 78.75) (width 0.2) (layer "F.Cu") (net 6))
 (segment (start 104.5 73.25) (end 103.719659 74.030341) (width 0.2) (layer "F.Cu") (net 6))
 (segment (start 101.404943 63.055) (end 104.5 66.150057) (width 0.2) (layer "F.Cu") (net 6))
 (segment (start 104.5 66.150057) (end 104.5 73.25) (width 0.2) (layer "F.Cu") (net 6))
 (segment (start 100.635 66.865) (end 101.857693 65.642307) (width 0.2) (layer "F.Cu") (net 9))
 (segment (start 102.5 74.46645) (end 102.5 76) (width 0.2) (layer "F.Cu") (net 9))
 (segment (start 103.142307 65.642307) (end 104 66.5) (width 0.2) (layer "F.Cu") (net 9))
 (segment (start 104 66.5) (end 104 72.96645) (width 0.2) (layer "F.Cu") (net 9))
 (segment (start 104 72.96645) (end 102.5 74.46645) (width 0.2) (layer "F.Cu") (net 9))
 (segment (start 97.85 66.865) (end 100.635 66.865) (width 0.2) (layer "F.Cu") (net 9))
 (segment (start 101.857693 65.642307) (end 103.142307 65.642307) (width 0.2) (layer "F.Cu") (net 9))
 (segment (start 101.825 64.325) (end 97.85 64.325) (width 0.2) (layer "F.Cu") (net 7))
 (segment (start 102.5 65) (end 101.825 64.325) (width 0.2) (layer "F.Cu") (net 7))
 (via (at 102.5 65) (size 0.6) (drill 0.4) (layers "F.Cu" "B.Cu") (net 7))
 (segment (start 102.75 64.25) (end 103.6 64.25) (width 0.2) (layer "B.Cu") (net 7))
 (segment (start 102.5 64.5) (end 102.75 64.25) (width 0.2) (layer "B.Cu") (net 7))
 (segment (start 102.5 65) (end 102.5 64.5) (width 0.2) (layer "B.Cu") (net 7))
 (segment (start 102.504245 66.243307) (end 100.612552 68.135) (width 0.2) (layer "F.Cu") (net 10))
 (segment (start 100.612552 68.135) (end 97.85 68.135) (width 0.2) (layer "F.Cu") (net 10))
 (via (at 102.504245 66.243307) (size 0.6) (drill 0.4) (layers "F.Cu" "B.Cu") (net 10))
 (segment (start 102.504245 66.243307) (end 103.010938 66.75) (width 0.2) (layer "B.Cu") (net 10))
 (segment (start 103.010938 66.75) (end 103.6 66.75) (width 0.2) (layer "B.Cu") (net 10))
 (segment (start 102.504245 68.743307) (end 100.572552 70.675) (width 0.2) (layer "F.Cu") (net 12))
 (segment (start 100.572552 70.675) (end 97.85 70.675) (width 0.2) (layer "F.Cu") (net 12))
 (via (at 102.504245 68.743307) (size 0.6) (drill 0.4) (layers "F.Cu" "B.Cu") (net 12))
 (segment (start 102.504245 68.743307) (end 103.010938 69.25) (width 0.2) (layer "B.Cu") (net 12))
 (segment (start 103.010938 69.25) (end 103.6 69.25) (width 0.2) (layer "B.Cu") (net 12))
 (segment (start 99.883529 73.215) (end 97.85 73.215) (width 0.2) (layer "F.Cu") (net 14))
 (segment (start 101.848529 71.25) (end 99.883529 73.215) (width 0.2) (layer "F.Cu") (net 14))
 (segment (start 102.526534 71.25) (end 101.848529 71.25) (width 0.2) (layer "F.Cu") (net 14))
 (via (at 102.526534 71.25) (size 0.6) (drill 0.4) (layers "F.Cu" "B.Cu") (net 14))
 (segment (start 102.526534 71.25) (end 103.026534 71.75) (width 0.2) (layer "B.Cu") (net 14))
 (segment (start 103.026534 71.75) (end 103.6 71.75) (width 0.2) (layer "B.Cu") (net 14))
 (segment (start 99.905 65.595) (end 97.85 65.595) (width 0.2) (layer "F.Cu") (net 8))
 (segment (start 100.771197 65.511874) (end 99.988126 65.511874) (width 0.2) (layer "F.Cu") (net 8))
 (segment (start 99.988126 65.511874) (end 99.905 65.595) (width 0.2) (layer "F.Cu") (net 8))
 (via (at 100.771197 65.511874) (size 0.6) (drill 0.4) (layers "F.Cu" "B.Cu") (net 8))
 (segment (start 100.771197 65.511874) (end 101.038126 65.511874) (width 0.2) (layer "B.Cu") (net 8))
 (segment (start 101.038126 65.511874) (end 101.4 65.15) (width 0.2) (layer "B.Cu") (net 8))
 (segment (start 101.4 65.15) (end 101.4 64.25) (width 0.2) (layer "B.Cu") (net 8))
 (segment (start 100.345 69.405) (end 97.85 69.405) (width 0.2) (layer "F.Cu") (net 11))
 (segment (start 102.5 67.25) (end 100.345 69.405) (width 0.2) (layer "F.Cu") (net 11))
 (via (at 102.5 67.25) (size 0.6) (drill 0.4) (layers "F.Cu" "B.Cu") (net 11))
 (segment (start 102 66.75) (end 101.4 66.75) (width 0.2) (layer "B.Cu") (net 11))
 (segment (start 102.5 67.25) (end 102 66.75) (width 0.2) (layer "B.Cu") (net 11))
 (segment (start 100.305 71.945) (end 97.85 71.945) (width 0.2) (layer "F.Cu") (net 13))
 (segment (start 102.5 69.75) (end 100.305 71.945) (width 0.2) (layer "F.Cu") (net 13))
 (via (at 102.5 69.75) (size 0.6) (drill 0.4) (layers "F.Cu" "B.Cu") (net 13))
 (segment (start 102 69.25) (end 101.4 69.25) (width 0.2) (layer "B.Cu") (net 13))
 (segment (start 102.5 69.75) (end 102 69.25) (width 0.2) (layer "B.Cu") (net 13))
 (segment (start 105.5 73.215) (end 107.15 73.215) (width 0.2) (layer "F.Cu") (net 15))
 (via (at 105.5 73.215) (size 0.6) (drill 0.4) (layers "F.Cu" "B.Cu") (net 15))
 (segment (start 103.59 73.215) (end 102.125 71.75) (width 0.2) (layer "B.Cu") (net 15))
 (segment (start 105.5 73.215) (end 103.59 73.215) (width 0.2) (layer "B.Cu") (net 15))
 (segment (start 102.125 71.75) (end 101.4 71.75) (width 0.2) (layer "B.Cu") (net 15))
 (segment (start 104.25 63.4329) (end 105.1421 64.325) (width 0.2) (layer "F.Cu") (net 22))
 (segment (start 104.25 62.25) (end 104.25 63.4329) (width 0.2) (layer "F.Cu") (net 22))
 (segment (start 105.1421 64.325) (end 107.15 64.325) (width 0.2) (layer "F.Cu") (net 22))
 (via (at 104.25 62.25) (size 0.6) (drill 0.4) (layers "F.Cu" "B.Cu") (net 22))
 (segment (start 104.25 62.25) (end 103.75 62.25) (width 0.2) (layer "B.Cu") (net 22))
 (segment (start 103.6 62.1) (end 103.6 61) (width 0.2) (layer "B.Cu") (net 22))
 (segment (start 103.75 62.25) (end 103.6 62.1) (width 0.2) (layer "B.Cu") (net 22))
 (segment (start 100.75 62.25) (end 101.25 62.25) (width 0.2) (layer "F.Cu") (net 20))
 (segment (start 105.865 66.865) (end 107.15 66.865) (width 0.2) (layer "F.Cu") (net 20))
 (segment (start 101.25 62.25) (end 105.865 66.865) (width 0.2) (layer "F.Cu") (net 20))
 (via (at 100.75 62.25) (size 0.6) (drill 0.4) (layers "F.Cu" "B.Cu") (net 20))
 (segment (start 100.75 62.25) (end 100.75 61) (width 0.2) (layer "B.Cu") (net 20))
 (segment (start 102.5 53) (end 102.5 54.75) (width 0.2) (layer "B.Cu") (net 24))
 (segment (start 103.4125 55.6625) (end 103.4125 56.75) (width 0.2) (layer "B.Cu") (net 24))
 (segment (start 102.5 54.75) (end 103.4125 55.6625) (width 0.2) (layer "B.Cu") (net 24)))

